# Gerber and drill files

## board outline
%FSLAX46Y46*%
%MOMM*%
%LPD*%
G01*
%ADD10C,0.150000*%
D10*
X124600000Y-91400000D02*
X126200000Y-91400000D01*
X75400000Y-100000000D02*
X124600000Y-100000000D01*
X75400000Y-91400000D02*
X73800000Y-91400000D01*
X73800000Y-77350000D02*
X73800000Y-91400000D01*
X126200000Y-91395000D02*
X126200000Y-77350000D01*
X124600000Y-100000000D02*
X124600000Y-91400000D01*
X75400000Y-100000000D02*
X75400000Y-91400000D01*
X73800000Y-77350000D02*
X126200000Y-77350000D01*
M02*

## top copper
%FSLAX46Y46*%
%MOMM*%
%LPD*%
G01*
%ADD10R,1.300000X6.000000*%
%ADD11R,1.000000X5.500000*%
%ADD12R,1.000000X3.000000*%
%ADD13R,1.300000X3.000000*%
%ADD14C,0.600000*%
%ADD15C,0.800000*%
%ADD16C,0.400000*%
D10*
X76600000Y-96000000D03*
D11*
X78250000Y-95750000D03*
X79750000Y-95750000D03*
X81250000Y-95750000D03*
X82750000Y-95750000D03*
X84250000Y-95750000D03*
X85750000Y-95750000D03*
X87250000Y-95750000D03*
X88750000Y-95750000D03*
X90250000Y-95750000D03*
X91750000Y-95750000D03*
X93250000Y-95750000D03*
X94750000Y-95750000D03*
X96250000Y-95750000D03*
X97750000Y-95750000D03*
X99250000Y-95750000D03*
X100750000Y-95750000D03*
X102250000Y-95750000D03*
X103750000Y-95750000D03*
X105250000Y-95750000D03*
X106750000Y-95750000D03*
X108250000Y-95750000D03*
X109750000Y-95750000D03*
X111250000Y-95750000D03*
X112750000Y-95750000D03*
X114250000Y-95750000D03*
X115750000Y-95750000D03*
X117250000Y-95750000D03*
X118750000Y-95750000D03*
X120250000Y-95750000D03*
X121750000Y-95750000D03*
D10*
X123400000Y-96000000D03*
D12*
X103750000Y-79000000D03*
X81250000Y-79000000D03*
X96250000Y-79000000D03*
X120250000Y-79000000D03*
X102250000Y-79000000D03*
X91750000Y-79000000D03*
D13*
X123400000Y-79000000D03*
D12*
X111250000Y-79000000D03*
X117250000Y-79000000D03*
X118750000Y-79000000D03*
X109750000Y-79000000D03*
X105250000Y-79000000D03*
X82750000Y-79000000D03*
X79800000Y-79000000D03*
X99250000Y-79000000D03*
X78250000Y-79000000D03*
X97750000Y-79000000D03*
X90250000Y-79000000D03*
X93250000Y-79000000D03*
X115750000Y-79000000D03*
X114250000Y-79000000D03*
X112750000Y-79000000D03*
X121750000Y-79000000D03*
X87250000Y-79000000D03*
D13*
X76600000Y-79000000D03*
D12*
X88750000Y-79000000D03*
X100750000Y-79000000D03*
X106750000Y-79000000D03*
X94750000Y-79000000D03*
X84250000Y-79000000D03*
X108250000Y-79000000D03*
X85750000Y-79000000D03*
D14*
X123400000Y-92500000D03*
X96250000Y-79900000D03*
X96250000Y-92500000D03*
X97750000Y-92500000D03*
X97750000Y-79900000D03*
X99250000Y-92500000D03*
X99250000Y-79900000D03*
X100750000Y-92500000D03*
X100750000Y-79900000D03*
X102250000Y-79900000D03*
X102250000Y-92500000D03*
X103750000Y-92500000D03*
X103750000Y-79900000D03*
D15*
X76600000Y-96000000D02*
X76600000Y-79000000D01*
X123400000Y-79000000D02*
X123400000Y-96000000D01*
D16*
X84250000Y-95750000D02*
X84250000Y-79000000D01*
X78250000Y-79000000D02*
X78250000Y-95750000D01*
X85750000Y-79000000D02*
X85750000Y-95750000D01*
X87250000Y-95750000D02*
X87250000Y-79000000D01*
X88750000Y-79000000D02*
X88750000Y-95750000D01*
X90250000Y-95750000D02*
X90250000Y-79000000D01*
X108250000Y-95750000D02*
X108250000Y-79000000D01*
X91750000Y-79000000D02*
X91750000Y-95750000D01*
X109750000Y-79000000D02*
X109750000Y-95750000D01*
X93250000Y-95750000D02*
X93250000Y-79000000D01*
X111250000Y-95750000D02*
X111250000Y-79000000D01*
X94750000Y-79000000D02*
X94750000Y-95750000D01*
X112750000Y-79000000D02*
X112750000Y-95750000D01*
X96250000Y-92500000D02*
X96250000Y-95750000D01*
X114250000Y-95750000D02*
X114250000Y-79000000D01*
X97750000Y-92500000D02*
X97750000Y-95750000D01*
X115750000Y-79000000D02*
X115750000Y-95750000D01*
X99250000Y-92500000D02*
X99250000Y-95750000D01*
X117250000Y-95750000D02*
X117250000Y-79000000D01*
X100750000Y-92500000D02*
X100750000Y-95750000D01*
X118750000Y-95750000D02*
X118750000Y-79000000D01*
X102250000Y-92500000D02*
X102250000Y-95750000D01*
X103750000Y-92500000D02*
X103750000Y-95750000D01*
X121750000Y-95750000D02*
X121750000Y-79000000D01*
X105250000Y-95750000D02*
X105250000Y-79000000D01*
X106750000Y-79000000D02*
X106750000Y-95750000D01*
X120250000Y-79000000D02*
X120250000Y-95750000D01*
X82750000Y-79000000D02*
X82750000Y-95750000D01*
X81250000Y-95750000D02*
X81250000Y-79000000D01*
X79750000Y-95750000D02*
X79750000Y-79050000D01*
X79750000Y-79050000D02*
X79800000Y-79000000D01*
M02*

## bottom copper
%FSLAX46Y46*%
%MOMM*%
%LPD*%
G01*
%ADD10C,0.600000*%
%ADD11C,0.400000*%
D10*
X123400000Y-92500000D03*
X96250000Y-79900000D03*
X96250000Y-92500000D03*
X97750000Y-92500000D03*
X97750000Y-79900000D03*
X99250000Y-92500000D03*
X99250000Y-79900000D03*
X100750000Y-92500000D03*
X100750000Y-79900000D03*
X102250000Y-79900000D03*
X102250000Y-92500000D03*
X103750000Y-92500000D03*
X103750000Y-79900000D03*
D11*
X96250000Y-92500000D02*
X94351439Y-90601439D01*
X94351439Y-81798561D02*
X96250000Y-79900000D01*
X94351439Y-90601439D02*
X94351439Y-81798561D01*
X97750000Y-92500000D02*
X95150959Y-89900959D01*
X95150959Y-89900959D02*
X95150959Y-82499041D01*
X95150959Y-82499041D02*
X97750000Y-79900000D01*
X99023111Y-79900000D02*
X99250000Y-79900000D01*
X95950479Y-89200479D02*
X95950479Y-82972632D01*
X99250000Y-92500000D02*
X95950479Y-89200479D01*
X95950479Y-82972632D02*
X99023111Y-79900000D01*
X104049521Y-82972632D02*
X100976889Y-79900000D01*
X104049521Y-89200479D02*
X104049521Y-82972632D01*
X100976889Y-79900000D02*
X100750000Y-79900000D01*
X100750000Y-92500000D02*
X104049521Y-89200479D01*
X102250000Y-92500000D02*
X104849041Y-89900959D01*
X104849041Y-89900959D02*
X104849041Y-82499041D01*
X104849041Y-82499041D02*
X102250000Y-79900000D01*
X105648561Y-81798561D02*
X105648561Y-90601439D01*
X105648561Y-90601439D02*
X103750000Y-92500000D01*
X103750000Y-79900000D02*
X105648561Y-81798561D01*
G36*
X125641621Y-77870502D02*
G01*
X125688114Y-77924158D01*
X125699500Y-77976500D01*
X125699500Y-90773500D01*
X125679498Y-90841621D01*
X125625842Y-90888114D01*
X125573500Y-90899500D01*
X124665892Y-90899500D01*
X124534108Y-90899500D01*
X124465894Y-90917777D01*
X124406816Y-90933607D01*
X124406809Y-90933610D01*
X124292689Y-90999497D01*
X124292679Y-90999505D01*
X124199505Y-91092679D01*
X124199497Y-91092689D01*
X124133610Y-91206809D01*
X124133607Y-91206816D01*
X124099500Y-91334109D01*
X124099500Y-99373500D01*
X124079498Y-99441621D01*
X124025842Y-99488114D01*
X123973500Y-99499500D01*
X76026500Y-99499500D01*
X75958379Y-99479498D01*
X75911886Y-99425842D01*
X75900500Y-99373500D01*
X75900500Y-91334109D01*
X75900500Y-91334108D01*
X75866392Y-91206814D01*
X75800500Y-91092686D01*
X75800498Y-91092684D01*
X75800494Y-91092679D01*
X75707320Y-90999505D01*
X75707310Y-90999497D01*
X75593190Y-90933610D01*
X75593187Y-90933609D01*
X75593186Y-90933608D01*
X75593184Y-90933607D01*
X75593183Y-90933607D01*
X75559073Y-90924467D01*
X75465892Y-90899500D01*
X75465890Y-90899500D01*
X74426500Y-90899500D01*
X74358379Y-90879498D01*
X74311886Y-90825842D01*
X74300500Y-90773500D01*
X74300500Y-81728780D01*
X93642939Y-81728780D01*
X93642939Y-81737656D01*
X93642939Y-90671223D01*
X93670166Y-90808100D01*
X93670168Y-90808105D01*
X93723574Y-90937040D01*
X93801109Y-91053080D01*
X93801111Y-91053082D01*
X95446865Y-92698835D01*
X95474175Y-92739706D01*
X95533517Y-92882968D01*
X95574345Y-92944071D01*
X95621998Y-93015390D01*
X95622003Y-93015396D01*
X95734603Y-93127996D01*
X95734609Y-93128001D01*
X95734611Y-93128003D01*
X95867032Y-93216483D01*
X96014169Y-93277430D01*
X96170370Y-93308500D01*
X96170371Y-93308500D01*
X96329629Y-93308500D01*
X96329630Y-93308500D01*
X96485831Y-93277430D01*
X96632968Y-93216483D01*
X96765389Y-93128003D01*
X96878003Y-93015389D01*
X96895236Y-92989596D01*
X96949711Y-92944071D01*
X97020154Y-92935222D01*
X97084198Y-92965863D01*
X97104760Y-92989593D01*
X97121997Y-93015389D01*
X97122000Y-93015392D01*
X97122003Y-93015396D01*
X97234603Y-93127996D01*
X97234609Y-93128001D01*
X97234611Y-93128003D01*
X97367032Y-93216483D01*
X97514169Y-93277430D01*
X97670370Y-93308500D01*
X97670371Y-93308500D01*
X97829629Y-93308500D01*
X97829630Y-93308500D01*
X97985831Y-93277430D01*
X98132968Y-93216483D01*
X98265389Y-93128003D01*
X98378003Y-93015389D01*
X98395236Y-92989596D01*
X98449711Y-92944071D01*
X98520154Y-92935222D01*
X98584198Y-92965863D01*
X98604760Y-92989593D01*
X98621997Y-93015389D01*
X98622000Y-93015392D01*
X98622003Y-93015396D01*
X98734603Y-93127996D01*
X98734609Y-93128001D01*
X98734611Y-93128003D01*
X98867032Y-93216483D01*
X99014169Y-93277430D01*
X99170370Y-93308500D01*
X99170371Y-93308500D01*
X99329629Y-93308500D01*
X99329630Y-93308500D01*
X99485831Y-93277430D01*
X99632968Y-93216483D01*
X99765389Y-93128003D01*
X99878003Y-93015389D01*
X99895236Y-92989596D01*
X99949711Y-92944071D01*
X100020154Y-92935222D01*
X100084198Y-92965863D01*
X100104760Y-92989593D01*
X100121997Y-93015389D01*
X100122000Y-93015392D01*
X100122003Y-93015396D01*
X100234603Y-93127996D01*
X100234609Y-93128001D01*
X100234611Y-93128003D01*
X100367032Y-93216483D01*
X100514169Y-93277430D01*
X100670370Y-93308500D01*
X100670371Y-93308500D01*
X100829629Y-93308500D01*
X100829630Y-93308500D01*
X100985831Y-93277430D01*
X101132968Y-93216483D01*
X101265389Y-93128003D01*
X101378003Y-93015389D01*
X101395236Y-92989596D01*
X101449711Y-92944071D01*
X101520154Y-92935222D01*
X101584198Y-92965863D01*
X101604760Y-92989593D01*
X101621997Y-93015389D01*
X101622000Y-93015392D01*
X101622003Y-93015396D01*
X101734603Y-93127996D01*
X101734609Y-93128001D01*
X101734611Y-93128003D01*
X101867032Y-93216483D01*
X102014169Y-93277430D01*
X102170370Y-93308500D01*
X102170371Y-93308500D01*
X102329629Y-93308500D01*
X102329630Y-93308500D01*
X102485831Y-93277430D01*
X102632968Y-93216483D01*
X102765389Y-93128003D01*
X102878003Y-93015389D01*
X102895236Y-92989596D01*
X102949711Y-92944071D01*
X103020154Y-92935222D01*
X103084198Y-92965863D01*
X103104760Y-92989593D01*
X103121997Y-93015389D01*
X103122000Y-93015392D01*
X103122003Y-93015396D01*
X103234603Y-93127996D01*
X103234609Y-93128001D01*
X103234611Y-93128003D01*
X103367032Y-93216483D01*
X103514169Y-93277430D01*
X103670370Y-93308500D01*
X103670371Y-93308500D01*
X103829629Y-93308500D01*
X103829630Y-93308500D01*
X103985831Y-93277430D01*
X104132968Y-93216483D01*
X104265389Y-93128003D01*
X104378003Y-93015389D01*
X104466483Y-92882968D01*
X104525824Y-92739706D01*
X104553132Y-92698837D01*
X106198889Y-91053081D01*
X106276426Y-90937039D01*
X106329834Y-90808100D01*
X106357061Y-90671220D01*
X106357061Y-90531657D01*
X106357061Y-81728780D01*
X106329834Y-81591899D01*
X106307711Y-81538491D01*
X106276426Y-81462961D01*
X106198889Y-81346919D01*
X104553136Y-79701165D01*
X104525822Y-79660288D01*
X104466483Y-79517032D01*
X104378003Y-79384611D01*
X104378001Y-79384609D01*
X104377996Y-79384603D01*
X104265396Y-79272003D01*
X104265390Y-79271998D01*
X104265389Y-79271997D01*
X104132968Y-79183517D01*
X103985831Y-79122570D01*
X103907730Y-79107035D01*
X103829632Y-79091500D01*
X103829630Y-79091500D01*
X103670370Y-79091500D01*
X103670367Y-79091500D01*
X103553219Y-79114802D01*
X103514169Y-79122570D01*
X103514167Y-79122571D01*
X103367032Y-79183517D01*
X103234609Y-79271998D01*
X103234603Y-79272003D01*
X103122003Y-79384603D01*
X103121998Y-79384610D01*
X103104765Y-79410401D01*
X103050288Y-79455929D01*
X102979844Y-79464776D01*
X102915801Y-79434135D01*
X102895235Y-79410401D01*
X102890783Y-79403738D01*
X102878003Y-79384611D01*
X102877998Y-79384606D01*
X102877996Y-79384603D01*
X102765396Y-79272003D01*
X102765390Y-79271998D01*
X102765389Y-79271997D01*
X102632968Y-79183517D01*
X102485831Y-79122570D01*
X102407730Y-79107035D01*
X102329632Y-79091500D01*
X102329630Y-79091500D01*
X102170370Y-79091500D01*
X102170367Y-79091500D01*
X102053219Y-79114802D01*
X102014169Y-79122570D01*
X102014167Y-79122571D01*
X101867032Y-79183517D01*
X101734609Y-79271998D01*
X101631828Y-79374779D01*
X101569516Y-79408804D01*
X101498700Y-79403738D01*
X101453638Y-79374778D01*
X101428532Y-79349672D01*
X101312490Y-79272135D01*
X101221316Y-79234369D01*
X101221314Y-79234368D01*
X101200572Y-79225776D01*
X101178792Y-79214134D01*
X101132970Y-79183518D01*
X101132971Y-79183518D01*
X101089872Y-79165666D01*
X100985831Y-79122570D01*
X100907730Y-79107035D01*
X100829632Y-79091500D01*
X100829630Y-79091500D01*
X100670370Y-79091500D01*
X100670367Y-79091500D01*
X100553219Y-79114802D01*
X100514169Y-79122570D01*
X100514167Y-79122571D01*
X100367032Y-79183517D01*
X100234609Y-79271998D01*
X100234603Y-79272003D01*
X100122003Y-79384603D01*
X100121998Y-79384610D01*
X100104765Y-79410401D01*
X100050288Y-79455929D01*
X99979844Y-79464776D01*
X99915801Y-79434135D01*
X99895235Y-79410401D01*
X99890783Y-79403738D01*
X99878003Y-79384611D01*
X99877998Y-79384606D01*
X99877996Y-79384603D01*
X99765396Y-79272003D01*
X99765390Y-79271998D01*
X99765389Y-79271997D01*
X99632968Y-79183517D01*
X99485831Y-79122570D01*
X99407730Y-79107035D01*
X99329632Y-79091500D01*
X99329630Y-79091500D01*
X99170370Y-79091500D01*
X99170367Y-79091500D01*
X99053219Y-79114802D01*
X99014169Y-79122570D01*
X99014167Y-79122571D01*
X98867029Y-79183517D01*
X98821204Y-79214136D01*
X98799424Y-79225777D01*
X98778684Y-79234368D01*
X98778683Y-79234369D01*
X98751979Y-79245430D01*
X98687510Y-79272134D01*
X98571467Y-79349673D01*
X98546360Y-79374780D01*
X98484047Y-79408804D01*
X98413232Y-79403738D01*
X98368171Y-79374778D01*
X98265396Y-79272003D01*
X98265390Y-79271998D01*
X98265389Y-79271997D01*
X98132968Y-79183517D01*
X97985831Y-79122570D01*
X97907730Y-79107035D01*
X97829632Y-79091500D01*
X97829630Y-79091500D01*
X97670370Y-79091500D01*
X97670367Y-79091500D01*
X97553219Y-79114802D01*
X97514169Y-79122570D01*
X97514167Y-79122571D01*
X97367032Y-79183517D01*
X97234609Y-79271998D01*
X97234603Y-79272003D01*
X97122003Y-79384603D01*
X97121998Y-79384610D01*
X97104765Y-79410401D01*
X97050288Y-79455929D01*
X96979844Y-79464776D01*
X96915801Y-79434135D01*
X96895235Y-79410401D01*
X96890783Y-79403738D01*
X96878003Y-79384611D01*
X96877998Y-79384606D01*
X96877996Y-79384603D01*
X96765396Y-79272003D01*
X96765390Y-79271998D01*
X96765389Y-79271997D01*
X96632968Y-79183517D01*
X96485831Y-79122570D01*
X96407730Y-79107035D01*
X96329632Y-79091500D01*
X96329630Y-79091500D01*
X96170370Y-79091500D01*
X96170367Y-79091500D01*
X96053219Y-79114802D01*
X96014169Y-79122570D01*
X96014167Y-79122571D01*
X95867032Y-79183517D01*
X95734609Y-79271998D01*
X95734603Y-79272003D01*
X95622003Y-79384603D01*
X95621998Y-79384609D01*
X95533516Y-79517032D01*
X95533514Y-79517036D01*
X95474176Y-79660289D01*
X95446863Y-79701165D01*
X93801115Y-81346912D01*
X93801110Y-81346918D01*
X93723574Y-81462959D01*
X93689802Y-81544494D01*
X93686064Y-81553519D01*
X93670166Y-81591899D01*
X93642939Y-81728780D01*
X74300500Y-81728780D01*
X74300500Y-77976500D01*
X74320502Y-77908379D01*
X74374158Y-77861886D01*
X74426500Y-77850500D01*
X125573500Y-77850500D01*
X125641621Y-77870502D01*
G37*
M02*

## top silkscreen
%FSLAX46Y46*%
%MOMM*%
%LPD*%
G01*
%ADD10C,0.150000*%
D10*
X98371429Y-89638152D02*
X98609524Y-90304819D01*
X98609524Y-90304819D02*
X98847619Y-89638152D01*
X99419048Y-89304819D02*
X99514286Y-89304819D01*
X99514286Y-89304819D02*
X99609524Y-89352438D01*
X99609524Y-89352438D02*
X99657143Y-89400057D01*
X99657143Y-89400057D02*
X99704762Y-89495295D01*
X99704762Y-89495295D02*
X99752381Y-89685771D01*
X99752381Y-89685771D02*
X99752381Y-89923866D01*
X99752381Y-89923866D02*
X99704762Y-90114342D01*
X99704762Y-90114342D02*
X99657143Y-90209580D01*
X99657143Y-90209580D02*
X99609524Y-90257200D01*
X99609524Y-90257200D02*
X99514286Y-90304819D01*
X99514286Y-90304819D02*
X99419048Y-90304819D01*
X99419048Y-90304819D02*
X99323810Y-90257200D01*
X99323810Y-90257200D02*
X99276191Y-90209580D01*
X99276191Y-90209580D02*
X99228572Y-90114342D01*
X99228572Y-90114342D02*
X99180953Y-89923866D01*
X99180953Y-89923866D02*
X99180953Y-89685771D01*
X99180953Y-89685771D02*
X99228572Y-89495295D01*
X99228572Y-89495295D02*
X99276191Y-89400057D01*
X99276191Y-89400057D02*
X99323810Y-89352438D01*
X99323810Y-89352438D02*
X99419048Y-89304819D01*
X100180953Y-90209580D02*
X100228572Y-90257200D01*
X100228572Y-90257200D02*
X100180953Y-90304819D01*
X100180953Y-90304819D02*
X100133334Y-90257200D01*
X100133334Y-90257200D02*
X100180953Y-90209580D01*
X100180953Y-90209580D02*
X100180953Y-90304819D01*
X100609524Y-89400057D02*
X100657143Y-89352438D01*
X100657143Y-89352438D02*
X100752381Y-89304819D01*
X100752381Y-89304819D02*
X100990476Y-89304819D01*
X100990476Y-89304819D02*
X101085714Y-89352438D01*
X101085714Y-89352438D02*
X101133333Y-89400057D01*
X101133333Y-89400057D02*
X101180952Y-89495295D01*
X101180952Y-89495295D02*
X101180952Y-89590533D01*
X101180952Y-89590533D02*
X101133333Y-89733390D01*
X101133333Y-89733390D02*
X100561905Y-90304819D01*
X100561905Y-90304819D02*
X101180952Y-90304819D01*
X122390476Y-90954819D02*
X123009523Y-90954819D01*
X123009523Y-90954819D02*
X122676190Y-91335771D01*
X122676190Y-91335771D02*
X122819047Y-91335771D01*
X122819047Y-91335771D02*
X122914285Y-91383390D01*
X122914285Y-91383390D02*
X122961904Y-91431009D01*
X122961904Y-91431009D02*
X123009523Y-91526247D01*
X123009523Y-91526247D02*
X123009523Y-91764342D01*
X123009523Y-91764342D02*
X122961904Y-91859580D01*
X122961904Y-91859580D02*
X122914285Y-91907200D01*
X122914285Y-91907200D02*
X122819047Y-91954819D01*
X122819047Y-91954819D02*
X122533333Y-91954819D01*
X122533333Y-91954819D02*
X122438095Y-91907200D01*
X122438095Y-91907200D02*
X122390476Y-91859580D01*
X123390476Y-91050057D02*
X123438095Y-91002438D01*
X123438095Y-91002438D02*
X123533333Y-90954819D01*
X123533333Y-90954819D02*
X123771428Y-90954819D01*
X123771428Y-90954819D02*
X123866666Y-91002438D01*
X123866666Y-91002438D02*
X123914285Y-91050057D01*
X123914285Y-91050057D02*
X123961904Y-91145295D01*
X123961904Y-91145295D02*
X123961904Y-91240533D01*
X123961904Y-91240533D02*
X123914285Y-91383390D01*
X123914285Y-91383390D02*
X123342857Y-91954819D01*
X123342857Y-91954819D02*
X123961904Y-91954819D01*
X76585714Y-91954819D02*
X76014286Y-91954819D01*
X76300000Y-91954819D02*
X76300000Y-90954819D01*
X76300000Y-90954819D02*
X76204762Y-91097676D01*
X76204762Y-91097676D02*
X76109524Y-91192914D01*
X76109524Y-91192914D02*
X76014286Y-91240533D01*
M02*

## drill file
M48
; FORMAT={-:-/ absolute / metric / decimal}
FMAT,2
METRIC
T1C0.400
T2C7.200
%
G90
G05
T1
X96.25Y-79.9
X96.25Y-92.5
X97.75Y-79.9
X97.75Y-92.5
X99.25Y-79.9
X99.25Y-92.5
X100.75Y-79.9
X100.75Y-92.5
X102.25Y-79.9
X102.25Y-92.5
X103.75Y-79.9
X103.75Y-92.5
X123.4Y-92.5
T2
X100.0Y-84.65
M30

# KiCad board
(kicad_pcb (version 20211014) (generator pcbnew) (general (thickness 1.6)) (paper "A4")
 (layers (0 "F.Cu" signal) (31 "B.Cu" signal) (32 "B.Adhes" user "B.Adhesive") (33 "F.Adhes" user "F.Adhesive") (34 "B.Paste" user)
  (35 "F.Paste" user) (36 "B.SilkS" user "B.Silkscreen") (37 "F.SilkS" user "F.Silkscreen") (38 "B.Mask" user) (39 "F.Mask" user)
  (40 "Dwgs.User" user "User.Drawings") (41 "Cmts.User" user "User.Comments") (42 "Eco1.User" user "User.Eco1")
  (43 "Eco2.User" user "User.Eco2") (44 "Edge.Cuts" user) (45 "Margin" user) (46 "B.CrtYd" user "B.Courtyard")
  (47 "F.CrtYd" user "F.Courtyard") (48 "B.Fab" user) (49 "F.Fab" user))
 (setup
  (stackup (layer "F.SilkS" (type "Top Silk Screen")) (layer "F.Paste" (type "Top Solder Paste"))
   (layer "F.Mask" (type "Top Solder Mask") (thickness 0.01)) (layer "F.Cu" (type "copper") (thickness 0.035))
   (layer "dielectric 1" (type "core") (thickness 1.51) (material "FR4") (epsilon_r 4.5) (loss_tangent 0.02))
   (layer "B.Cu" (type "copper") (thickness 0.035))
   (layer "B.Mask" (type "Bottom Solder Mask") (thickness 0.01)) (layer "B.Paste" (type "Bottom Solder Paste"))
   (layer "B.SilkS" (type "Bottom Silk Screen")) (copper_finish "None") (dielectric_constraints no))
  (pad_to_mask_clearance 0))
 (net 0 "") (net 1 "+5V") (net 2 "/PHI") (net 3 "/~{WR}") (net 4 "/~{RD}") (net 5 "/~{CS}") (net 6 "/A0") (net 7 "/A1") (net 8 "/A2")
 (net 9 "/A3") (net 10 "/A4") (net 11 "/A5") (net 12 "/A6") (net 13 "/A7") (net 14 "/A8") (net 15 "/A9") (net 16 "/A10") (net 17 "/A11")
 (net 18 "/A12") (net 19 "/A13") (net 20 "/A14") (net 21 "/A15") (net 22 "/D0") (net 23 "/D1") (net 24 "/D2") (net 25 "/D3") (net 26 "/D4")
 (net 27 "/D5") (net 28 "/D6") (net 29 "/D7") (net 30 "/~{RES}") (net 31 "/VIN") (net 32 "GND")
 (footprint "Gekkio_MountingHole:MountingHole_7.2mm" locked (layer "F.Cu") (at 100 84.65)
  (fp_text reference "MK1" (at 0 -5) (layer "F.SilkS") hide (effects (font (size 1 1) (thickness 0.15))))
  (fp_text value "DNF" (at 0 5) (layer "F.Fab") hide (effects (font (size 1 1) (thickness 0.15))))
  (pad "" np_thru_hole circle locked (at 0 0) (size 7.2 7.2) (drill 7.2) (layers *.Cu *.Mask)))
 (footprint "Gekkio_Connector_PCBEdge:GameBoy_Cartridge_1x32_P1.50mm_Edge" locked (layer "F.Cu") (at 100 96)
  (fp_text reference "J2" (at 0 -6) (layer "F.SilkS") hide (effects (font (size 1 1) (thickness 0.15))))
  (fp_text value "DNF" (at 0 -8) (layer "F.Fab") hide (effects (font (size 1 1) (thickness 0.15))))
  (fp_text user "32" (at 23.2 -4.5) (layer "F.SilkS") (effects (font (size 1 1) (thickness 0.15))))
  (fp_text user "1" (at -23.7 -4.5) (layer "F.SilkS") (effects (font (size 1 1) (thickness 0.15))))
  (pad "1" connect rect locked (at -23.4 0 90) (size 6 1.3) (layers "F.Cu" "F.Mask") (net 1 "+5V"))
  (pad "2" connect rect locked (at -21.75 -0.25 90) (size 5.5 1) (layers "F.Cu" "F.Mask") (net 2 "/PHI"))
  (pad "3" connect rect locked (at -20.25 -0.25 90) (size 5.5 1) (layers "F.Cu" "F.Mask") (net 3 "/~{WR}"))
  (pad "4" connect rect locked (at -18.75 -0.25 90) (size 5.5 1) (layers "F.Cu" "F.Mask") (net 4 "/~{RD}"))
  (pad "5" connect rect locked (at -17.25 -0.25 90) (size 5.5 1) (layers "F.Cu" "F.Mask") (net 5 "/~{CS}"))
  (pad "6" connect rect locked (at -15.75 -0.25 90) (size 5.5 1) (layers "F.Cu" "F.Mask") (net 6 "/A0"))
  (pad "7" connect rect locked (at -14.25 -0.25 90) (size 5.5 1) (layers "F.Cu" "F.Mask") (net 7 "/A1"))
  (pad "8" connect rect locked (at -12.75 -0.25 90) (size 5.5 1) (layers "F.Cu" "F.Mask") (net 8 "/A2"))
  (pad "9" connect rect locked (at -11.25 -0.25 90) (size 5.5 1) (layers "F.Cu" "F.Mask") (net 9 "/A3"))
  (pad "10" connect rect locked (at -9.75 -0.25 90) (size 5.5 1) (layers "F.Cu" "F.Mask") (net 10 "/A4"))
  (pad "11" connect rect locked (at -8.25 -0.25 90) (size 5.5 1) (layers "F.Cu" "F.Mask") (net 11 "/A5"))
  (pad "12" connect rect locked (at -6.75 -0.25 90) (size 5.5 1) (layers "F.Cu" "F.Mask") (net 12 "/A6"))
  (pad "13" connect rect locked (at -5.25 -0.25 90) (size 5.5 1) (layers "F.Cu" "F.Mask") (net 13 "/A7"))
  (pad "14" connect rect locked (at -3.75 -0.25 90) (size 5.5 1) (layers "F.Cu" "F.Mask") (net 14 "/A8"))
  (pad "15" connect rect locked (at -2.25 -0.25 90) (size 5.5 1) (layers "F.Cu" "F.Mask") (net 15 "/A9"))
  (pad "16" connect rect locked (at -0.75 -0.25 90) (size 5.5 1) (layers "F.Cu" "F.Mask") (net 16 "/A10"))
  (pad "17" connect rect locked (at 0.75 -0.25 90) (size 5.5 1) (layers "F.Cu" "F.Mask") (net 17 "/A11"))
  (pad "18" connect rect locked (at 2.25 -0.25 90) (size 5.5 1) (layers "F.Cu" "F.Mask") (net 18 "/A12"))
  (pad "19" connect rect locked (at 3.75 -0.25 90) (size 5.5 1) (layers "F.Cu" "F.Mask") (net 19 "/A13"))
  (pad "20" connect rect locked (at 5.25 -0.25 90) (size 5.5 1) (layers "F.Cu" "F.Mask") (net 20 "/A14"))
  (pad "21" connect rect locked (at 6.75 -0.25 90) (size 5.5 1) (layers "F.Cu" "F.Mask") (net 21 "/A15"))
  (pad "22" connect rect locked (at 8.25 -0.25 90) (size 5.5 1) (layers "F.Cu" "F.Mask") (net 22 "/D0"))
  (pad "23" connect rect locked (at 9.75 -0.25 90) (size 5.5 1) (layers "F.Cu" "F.Mask") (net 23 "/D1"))
  (pad "24" connect rect locked (at 11.25 -0.25 90) (size 5.5 1) (layers "F.Cu" "F.Mask") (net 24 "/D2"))
  (pad "25" connect rect locked (at 12.75 -0.25 90) (size 5.5 1) (layers "F.Cu" "F.Mask") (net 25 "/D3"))
  (pad "26" connect rect locked (at 14.25 -0.25 90) (size 5.5 1) (layers "F.Cu" "F.Mask") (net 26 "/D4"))
  (pad "27" connect rect locked (at 15.75 -0.25 90) (size 5.5 1) (layers "F.Cu" "F.Mask") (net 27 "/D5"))
  (pad "28" connect rect locked (at 17.25 -0.25 90) (size 5.5 1) (layers "F.Cu" "F.Mask") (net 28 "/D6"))
  (pad "29" connect rect locked (at 18.75 -0.25 90) (size 5.5 1) (layers "F.Cu" "F.Mask") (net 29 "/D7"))
  (pad "30" connect rect locked (at 20.25 -0.25 90) (size 5.5 1) (layers "F.Cu" "F.Mask") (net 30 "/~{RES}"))
  (pad "31" connect rect locked (at 21.75 -0.25 90) (size 5.5 1) (layers "F.Cu" "F.Mask") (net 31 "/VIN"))
  (pad "32" connect rect locked (at 23.4 0 90) (size 6 1.3) (layers "F.Cu" "F.Mask") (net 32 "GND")))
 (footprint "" (layer "F.Cu") (at 103.75 79)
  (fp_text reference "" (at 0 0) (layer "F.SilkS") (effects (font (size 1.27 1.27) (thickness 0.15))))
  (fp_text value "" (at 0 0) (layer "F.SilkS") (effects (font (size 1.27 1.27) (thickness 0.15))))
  (pad "19" connect rect locked (at 0 0 90) (size 3 1) (layers "F.Cu" "F.Mask") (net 19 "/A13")))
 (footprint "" (layer "F.Cu") (at 81.25 79)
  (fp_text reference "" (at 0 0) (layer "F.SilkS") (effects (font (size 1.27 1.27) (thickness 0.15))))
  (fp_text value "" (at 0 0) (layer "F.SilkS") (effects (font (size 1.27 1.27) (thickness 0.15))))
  (pad "4" connect rect locked (at 0 0 90) (size 3 1) (layers "F.Cu" "F.Mask") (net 4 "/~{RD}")))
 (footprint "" (layer "F.Cu") (at 96.25 79)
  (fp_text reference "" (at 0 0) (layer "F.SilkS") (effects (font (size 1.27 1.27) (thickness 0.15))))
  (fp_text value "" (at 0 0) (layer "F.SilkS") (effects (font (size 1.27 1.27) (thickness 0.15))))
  (pad "14" connect rect locked (at 0 0 90) (size 3 1) (layers "F.Cu" "F.Mask") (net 14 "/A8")))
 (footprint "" (layer "F.Cu") (at 120.25 79)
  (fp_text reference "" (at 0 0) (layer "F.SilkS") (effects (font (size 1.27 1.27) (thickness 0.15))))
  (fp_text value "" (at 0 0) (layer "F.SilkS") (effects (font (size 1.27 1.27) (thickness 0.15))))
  (pad "30" connect rect locked (at 0 0 90) (size 3 1) (layers "F.Cu" "F.Mask") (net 30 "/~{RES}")))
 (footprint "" (layer "F.Cu") (at 102.25 79)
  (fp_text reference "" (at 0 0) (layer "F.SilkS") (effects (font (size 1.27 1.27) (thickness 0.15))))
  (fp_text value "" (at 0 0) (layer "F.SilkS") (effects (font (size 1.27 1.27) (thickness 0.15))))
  (pad "18" connect rect locked (at 0 0 90) (size 3 1) (layers "F.Cu" "F.Mask") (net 18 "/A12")))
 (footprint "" (layer "F.Cu") (at 91.75 79)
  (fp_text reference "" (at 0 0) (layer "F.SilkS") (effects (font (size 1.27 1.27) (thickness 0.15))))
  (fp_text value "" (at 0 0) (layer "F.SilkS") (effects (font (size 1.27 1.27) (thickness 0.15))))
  (pad "11" connect rect locked (at 0 0 90) (size 3 1) (layers "F.Cu" "F.Mask") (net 11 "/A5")))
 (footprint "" (layer "F.Cu") (at 123.4 79)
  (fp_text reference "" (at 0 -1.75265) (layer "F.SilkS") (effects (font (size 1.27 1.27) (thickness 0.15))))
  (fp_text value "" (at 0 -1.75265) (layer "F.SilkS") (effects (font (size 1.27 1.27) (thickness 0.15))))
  (pad "32" connect rect locked (at 0 0 90) (size 3 1.3) (layers "F.Cu" "F.Mask") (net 32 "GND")))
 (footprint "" (layer "F.Cu") (at 111.25 79)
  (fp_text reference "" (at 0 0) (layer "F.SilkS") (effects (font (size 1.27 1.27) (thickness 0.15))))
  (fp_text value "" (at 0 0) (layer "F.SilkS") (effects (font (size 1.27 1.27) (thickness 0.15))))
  (pad "24" connect rect locked (at 0 0 90) (size 3 1) (layers "F.Cu" "F.Mask") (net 24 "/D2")))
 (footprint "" (layer "F.Cu") (at 117.25 79)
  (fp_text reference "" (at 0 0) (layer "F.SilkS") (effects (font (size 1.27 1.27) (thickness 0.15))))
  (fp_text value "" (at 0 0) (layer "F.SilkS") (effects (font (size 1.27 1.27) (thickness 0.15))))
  (pad "28" connect rect locked (at 0 0 90) (size 3 1) (layers "F.Cu" "F.Mask") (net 28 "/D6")))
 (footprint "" (layer "F.Cu") (at 118.75 79)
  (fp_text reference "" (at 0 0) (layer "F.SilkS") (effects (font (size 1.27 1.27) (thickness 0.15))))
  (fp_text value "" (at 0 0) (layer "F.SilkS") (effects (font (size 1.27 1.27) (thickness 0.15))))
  (pad "29" connect rect locked (at 0 0 90) (size 3 1) (layers "F.Cu" "F.Mask") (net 29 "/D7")))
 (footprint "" (layer "F.Cu") (at 109.75 79)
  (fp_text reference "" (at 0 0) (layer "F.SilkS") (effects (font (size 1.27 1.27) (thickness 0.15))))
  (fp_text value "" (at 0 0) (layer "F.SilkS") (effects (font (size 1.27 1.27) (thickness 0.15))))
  (pad "23" connect rect locked (at 0 0 90) (size 3 1) (layers "F.Cu" "F.Mask") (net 23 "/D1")))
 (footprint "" (layer "F.Cu") (at 105.25 79)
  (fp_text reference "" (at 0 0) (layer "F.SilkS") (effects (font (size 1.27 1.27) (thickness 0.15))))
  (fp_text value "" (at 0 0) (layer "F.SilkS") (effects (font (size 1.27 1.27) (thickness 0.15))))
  (pad "20" connect rect locked (at 0 0 90) (size 3 1) (layers "F.Cu" "F.Mask") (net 20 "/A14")))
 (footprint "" (layer "F.Cu") (at 82.75 79)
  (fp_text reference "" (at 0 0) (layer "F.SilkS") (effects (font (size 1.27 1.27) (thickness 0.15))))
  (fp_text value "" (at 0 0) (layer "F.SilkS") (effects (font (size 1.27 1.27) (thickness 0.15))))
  (pad "5" connect rect locked (at 0 0 90) (size 3 1) (layers "F.Cu" "F.Mask") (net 5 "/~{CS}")))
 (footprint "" (layer "F.Cu") (at 79.8 79)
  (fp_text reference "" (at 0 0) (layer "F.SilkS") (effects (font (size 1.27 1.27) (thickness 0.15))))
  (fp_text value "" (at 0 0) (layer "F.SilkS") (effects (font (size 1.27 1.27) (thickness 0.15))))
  (pad "3" connect rect locked (at 0 0 90) (size 3 1) (layers "F.Cu" "F.Mask") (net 3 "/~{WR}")))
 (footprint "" (layer "F.Cu") (at 99.25 79)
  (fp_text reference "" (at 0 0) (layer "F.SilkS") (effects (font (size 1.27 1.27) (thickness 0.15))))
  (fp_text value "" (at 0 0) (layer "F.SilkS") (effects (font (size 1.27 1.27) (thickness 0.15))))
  (pad "16" connect rect locked (at 0 0 90) (size 3 1) (layers "F.Cu" "F.Mask") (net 16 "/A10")))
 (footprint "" (layer "F.Cu") (at 78.25 79)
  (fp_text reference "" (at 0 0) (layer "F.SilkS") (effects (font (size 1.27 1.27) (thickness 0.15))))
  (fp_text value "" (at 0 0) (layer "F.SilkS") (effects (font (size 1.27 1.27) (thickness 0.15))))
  (pad "2" connect rect locked (at 0 0 90) (size 3 1) (layers "F.Cu" "F.Mask") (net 2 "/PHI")))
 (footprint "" (layer "F.Cu") (at 97.75 79)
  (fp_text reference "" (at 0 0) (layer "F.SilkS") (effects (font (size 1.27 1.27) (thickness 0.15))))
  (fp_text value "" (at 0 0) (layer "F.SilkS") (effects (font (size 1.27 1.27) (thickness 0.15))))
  (pad "15" connect rect locked (at 0 0 90) (size 3 1) (layers "F.Cu" "F.Mask") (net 15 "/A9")))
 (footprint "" (layer "F.Cu") (at 90.25 79)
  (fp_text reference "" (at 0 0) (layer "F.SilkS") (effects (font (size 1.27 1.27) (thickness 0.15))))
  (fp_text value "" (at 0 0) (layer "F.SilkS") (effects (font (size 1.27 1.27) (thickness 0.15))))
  (pad "10" connect rect locked (at 0 0 90) (size 3 1) (layers "F.Cu" "F.Mask") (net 10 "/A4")))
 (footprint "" (layer "F.Cu") (at 93.25 79)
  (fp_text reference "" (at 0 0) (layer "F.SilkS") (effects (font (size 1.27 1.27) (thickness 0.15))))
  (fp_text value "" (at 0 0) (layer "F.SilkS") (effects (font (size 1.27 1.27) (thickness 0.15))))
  (pad "12" connect rect locked (at 0 0 90) (size 3 1) (layers "F.Cu" "F.Mask") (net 12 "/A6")))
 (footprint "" (layer "F.Cu") (at 115.75 79)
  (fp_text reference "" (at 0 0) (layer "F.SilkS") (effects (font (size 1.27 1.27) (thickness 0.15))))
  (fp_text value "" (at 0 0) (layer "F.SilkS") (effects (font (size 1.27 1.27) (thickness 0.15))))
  (pad "27" connect rect locked (at 0 0 90) (size 3 1) (layers "F.Cu" "F.Mask") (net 27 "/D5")))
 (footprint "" (layer "F.Cu") (at 114.25 79)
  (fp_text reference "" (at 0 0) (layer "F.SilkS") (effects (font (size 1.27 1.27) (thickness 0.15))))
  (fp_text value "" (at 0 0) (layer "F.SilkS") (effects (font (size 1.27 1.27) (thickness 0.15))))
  (pad "26" connect rect locked (at 0 0 90) (size 3 1) (layers "F.Cu" "F.Mask") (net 26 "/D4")))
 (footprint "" (layer "F.Cu") (at 112.75 79)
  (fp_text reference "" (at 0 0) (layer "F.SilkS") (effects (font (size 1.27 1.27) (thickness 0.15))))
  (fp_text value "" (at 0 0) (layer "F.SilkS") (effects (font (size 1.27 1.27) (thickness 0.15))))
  (pad "25" connect rect locked (at 0 0 90) (size 3 1) (layers "F.Cu" "F.Mask") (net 25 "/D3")))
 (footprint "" (layer "F.Cu") (at 121.75 79)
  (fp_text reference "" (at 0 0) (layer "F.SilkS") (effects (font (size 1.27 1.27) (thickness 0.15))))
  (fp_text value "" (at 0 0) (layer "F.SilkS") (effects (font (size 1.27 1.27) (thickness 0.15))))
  (pad "31" connect rect locked (at 0 0 90) (size 3 1) (layers "F.Cu" "F.Mask") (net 31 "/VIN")))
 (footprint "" (layer "F.Cu") (at 87.25 79)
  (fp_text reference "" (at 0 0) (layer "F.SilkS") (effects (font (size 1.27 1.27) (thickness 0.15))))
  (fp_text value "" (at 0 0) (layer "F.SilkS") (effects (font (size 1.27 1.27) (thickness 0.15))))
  (pad "8" connect rect locked (at 0 0 90) (size 3 1) (layers "F.Cu" "F.Mask") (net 8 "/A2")))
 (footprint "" (layer "F.Cu") (at 76.6 79)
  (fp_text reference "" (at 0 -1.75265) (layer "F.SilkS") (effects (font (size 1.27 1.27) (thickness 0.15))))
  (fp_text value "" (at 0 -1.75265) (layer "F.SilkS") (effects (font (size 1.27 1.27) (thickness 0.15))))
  (pad "1" connect rect locked (at 0 0 90) (size 3 1.3) (layers "F.Cu" "F.Mask") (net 1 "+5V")))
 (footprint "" (layer "F.Cu") (at 88.75 79)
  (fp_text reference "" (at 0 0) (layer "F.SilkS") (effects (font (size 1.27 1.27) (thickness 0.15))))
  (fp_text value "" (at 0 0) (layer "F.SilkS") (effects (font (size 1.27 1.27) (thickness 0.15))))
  (pad "9" connect rect locked (at 0 0 90) (size 3 1) (layers "F.Cu" "F.Mask") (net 9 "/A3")))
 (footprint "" (layer "F.Cu") (at 100.75 79)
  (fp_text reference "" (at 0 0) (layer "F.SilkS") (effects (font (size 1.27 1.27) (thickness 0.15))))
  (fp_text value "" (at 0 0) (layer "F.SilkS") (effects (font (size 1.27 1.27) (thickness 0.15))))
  (pad "17" connect rect locked (at 0 0 90) (size 3 1) (layers "F.Cu" "F.Mask") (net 17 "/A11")))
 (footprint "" (layer "F.Cu") (at 106.75 79)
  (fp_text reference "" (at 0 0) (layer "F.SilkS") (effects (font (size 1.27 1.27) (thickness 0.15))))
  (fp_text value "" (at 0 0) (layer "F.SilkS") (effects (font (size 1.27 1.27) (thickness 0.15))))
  (pad "21" connect rect locked (at 0 0 90) (size 3 1) (layers "F.Cu" "F.Mask") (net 21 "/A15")))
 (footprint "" (layer "F.Cu") (at 94.75 79)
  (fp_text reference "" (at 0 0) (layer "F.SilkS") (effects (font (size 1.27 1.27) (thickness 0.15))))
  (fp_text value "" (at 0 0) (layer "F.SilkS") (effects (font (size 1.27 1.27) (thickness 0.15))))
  (pad "13" connect rect locked (at 0 0 90) (size 3 1) (layers "F.Cu" "F.Mask") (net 13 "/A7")))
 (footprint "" (layer "F.Cu") (at 84.25 79)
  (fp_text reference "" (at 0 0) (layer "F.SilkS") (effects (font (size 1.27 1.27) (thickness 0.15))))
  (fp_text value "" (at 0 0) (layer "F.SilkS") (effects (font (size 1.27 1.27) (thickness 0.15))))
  (pad "6" connect rect locked (at 0 0 90) (size 3 1) (layers "F.Cu" "F.Mask") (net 6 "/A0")))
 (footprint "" (layer "F.Cu") (at 108.25 79)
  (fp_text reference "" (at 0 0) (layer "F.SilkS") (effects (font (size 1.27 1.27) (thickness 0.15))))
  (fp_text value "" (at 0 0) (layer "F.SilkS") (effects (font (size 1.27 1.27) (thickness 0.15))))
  (pad "22" connect rect locked (at 0 0 90) (size 3 1) (layers "F.Cu" "F.Mask") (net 22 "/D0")))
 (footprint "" (layer "F.Cu") (at 85.75 79)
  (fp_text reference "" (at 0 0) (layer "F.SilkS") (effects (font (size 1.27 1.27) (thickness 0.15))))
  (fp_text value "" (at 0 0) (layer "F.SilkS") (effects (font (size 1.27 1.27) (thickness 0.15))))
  (pad "7" connect rect locked (at 0 0 90) (size 3 1) (layers "F.Cu" "F.Mask") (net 7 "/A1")))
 (gr_line (start 124.6 91.4) (end 126.2 91.4) (layer "Edge.Cuts") (width 0.15))
 (gr_line (start 75.4 100) (end 124.6 100) (layer "Edge.Cuts") (width 0.15))
 (gr_line (start 75.4 91.4) (end 73.8 91.4) (layer "Edge.Cuts") (width 0.15))
 (gr_line (start 73.8 77.35) (end 73.8 91.4) (layer "Edge.Cuts") (width 0.15))
 (gr_line (start 126.2 91.395) (end 126.2 77.35) (layer "Edge.Cuts") (width 0.15))
 (gr_line (start 124.6 100) (end 124.6 91.4) (layer "Edge.Cuts") (width 0.15))
 (gr_line (start 75.4 100) (end 75.4 91.4) (layer "Edge.Cuts") (width 0.15))
 (gr_line (start 73.8 77.35) (end 126.2 77.35) (layer "Edge.Cuts") (width 0.15))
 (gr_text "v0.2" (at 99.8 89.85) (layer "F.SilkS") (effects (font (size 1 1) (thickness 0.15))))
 (segment (start 76.6 96) (end 76.6 79) (width 0.8) (layer "F.Cu") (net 1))
 (segment (start 123.4 79) (end 123.4 96) (width 0.8) (layer "F.Cu") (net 32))
 (via (at 123.4 92.5) (size 0.6) (drill 0.4) (layers "F.Cu" "B.Cu") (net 32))
 (segment (start 84.25 95.75) (end 84.25 79) (width 0.4) (layer "F.Cu") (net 6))
 (segment (start 78.25 79) (end 78.25 95.75) (width 0.4) (layer "F.Cu") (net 2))
 (segment (start 85.75 79) (end 85.75 95.75) (width 0.4) (layer "F.Cu") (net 7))
 (segment (start 87.25 95.75) (end 87.25 79) (width 0.4) (layer "F.Cu") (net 8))
 (segment (start 88.75 79) (end 88.75 95.75) (width 0.4) (layer "F.Cu") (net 9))
 (segment (start 90.25 95.75) (end 90.25 79) (width 0.4) (layer "F.Cu") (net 10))
 (segment (start 108.25 95.75) (end 108.25 79) (width 0.4) (layer "F.Cu") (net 22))
 (segment (start 91.75 79) (end 91.75 95.75) (width 0.4) (layer "F.Cu") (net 11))
 (segment (start 109.75 79) (end 109.75 95.75) (width 0.4) (layer "F.Cu") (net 23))
 (segment (start 93.25 95.75) (end 93.25 79) (width 0.4) (layer "F.Cu") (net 12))
 (segment (start 111.25 95.75) (end 111.25 79) (width 0.4) (layer "F.Cu") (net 24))
 (segment (start 94.75 79) (end 94.75 95.75) (width 0.4) (layer "F.Cu") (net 13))
 (segment (start 112.75 79) (end 112.75 95.75) (width 0.4) (layer "F.Cu") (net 25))
 (segment (start 96.25 92.5) (end 96.25 95.75) (width 0.4) (layer "F.Cu") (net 14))
 (via (at 96.25 79.9) (size 0.6) (drill 0.4) (layers "F.Cu" "B.Cu") (free) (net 14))
 (via (at 96.25 92.5) (size 0.6) (drill 0.4) (layers "F.Cu" "B.Cu") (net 14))
 (segment (start 96.25 92.5) (end 94.351439 90.601439) (width 0.4) (layer "B.Cu") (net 14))
 (segment (start 94.351439 81.798561) (end 96.25 79.9) (width 0.4) (layer "B.Cu") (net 14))
 (segment (start 94.351439 90.601439) (end 94.351439 81.798561) (width 0.4) (layer "B.Cu") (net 14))
 (segment (start 114.25 95.75) (end 114.25 79) (width 0.4) (layer "F.Cu") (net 26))
 (segment (start 97.75 92.5) (end 97.75 95.75) (width 0.4) (layer "F.Cu") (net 15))
 (via (at 97.75 92.5) (size 0.6) (drill 0.4) (layers "F.Cu" "B.Cu") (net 15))
 (via (at 97.75 79.9) (size 0.6) (drill 0.4) (layers "F.Cu" "B.Cu") (free) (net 15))
 (segment (start 97.75 92.5) (end 95.150959 89.900959) (width 0.4) (layer "B.Cu") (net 15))
 (segment (start 95.150959 89.900959) (end 95.150959 82.499041) (width 0.4) (layer "B.Cu") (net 15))
 (segment (start 95.150959 82.499041) (end 97.75 79.9) (width 0.4) (layer "B.Cu") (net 15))
 (segment (start 115.75 79) (end 115.75 95.75) (width 0.4) (layer "F.Cu") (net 27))
 (segment (start 99.25 92.5) (end 99.25 95.75) (width 0.4) (layer "F.Cu") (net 16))
 (via (at 99.25 92.5) (size 0.6) (drill 0.4) (layers "F.Cu" "B.Cu") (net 16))
 (via (at 99.25 79.9) (size 0.6) (drill 0.4) (layers "F.Cu" "B.Cu") (free) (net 16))
 (segment (start 99.023111 79.9) (end 99.25 79.9) (width 0.4) (layer "B.Cu") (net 16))
 (segment (start 95.950479 89.200479) (end 95.950479 82.972632) (width 0.4) (layer "B.Cu") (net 16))
 (segment (start 99.25 92.5) (end 95.950479 89.200479) (width 0.4) (layer "B.Cu") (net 16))
 (segment (start 95.950479 82.972632) (end 99.023111 79.9) (width 0.4) (layer "B.Cu") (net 16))
 (segment (start 117.25 95.75) (end 117.25 79) (width 0.4) (layer "F.Cu") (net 28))
 (segment (start 100.75 92.5) (end 100.75 95.75) (width 0.4) (layer "F.Cu") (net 17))
 (via (at 100.75 92.5) (size 0.6) (drill 0.4) (layers "F.Cu" "B.Cu") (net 17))
 (via (at 100.75 79.9) (size 0.6) (drill 0.4) (layers "F.Cu" "B.Cu") (free) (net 17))
 (segment (start 104.049521 82.972632) (end 100.976889 79.9) (width 0.4) (layer "B.Cu") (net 17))
 (segment (start 104.049521 89.200479) (end 104.049521 82.972632) (width 0.4) (layer "B.Cu") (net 17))
 (segment (start 100.976889 79.9) (end 100.75 79.9) (width 0.4) (layer "B.Cu") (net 17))
 (segment (start 100.75 92.5) (end 104.049521 89.200479) (width 0.4) (layer "B.Cu") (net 17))
 (segment (start 118.75 95.75) (end 118.75 79) (width 0.4) (layer "F.Cu") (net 29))
 (segment (start 102.25 92.5) (end 102.25 95.75) (width 0.4) (layer "F.Cu") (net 18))
 (via (at 102.25 79.9) (size 0.6) (drill 0.4) (layers "F.Cu" "B.Cu") (free) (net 18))
 (via (at 102.25 92.5) (size 0.6) (drill 0.4) (layers "F.Cu" "B.Cu") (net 18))
 (segment (start 102.25 92.5) (end 104.849041 89.900959) (width 0.4) (layer "B.Cu") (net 18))
 (segment (start 104.849041 89.900959) (end 104.849041 82.499041) (width 0.4) (layer "B.Cu") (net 18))
 (segment (start 104.849041 82.499041) (end 102.25 79.9) (width 0.4) (layer "B.Cu") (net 18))
 (segment (start 103.75 92.5) (end 103.75 95.75) (width 0.4) (layer "F.Cu") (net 19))
 (via (at 103.75 92.5) (size 0.6) (drill 0.4) (layers "F.Cu" "B.Cu") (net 19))
 (via (at 103.75 79.9) (size 0.6) (drill 0.4) (layers "F.Cu" "B.Cu") (free) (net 19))
 (segment (start 105.648561 81.798561) (end 105.648561 90.601439) (width 0.4) (layer "B.Cu") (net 19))
 (segment (start 105.648561 90.601439) (end 103.75 92.5) (width 0.4) (layer "B.Cu") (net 19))
 (segment (start 103.75 79.9) (end 105.648561 81.798561) (width 0.4) (layer "B.Cu") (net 19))
 (segment (start 121.75 95.75) (end 121.75 79) (width 0.4) (layer "F.Cu") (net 31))
 (segment (start 105.25 95.75) (end 105.25 79) (width 0.4) (layer "F.Cu") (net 20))
 (segment (start 106.75 79) (end 106.75 95.75) (width 0.4) (layer "F.Cu") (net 21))
 (segment (start 120.25 79) (end 120.25 95.75) (width 0.4) (layer "F.Cu") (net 30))
 (segment (start 82.75 79) (end 82.75 95.75) (width 0.4) (layer "F.Cu") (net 5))
 (segment (start 81.25 95.75) (end 81.25 79) (width 0.4) (layer "F.Cu") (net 4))
 (segment (start 79.75 95.75) (end 79.75 79.05) (width 0.4) (layer "F.Cu") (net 3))
 (segment (start 79.75 79.05) (end 79.8 79) (width 0.4) (layer "F.Cu") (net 3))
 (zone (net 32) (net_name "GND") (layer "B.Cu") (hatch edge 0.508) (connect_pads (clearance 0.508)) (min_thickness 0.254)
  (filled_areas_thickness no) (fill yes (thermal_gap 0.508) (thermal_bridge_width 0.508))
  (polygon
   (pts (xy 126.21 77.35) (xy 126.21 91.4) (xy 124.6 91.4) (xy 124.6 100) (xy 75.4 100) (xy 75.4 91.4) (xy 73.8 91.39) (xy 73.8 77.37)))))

